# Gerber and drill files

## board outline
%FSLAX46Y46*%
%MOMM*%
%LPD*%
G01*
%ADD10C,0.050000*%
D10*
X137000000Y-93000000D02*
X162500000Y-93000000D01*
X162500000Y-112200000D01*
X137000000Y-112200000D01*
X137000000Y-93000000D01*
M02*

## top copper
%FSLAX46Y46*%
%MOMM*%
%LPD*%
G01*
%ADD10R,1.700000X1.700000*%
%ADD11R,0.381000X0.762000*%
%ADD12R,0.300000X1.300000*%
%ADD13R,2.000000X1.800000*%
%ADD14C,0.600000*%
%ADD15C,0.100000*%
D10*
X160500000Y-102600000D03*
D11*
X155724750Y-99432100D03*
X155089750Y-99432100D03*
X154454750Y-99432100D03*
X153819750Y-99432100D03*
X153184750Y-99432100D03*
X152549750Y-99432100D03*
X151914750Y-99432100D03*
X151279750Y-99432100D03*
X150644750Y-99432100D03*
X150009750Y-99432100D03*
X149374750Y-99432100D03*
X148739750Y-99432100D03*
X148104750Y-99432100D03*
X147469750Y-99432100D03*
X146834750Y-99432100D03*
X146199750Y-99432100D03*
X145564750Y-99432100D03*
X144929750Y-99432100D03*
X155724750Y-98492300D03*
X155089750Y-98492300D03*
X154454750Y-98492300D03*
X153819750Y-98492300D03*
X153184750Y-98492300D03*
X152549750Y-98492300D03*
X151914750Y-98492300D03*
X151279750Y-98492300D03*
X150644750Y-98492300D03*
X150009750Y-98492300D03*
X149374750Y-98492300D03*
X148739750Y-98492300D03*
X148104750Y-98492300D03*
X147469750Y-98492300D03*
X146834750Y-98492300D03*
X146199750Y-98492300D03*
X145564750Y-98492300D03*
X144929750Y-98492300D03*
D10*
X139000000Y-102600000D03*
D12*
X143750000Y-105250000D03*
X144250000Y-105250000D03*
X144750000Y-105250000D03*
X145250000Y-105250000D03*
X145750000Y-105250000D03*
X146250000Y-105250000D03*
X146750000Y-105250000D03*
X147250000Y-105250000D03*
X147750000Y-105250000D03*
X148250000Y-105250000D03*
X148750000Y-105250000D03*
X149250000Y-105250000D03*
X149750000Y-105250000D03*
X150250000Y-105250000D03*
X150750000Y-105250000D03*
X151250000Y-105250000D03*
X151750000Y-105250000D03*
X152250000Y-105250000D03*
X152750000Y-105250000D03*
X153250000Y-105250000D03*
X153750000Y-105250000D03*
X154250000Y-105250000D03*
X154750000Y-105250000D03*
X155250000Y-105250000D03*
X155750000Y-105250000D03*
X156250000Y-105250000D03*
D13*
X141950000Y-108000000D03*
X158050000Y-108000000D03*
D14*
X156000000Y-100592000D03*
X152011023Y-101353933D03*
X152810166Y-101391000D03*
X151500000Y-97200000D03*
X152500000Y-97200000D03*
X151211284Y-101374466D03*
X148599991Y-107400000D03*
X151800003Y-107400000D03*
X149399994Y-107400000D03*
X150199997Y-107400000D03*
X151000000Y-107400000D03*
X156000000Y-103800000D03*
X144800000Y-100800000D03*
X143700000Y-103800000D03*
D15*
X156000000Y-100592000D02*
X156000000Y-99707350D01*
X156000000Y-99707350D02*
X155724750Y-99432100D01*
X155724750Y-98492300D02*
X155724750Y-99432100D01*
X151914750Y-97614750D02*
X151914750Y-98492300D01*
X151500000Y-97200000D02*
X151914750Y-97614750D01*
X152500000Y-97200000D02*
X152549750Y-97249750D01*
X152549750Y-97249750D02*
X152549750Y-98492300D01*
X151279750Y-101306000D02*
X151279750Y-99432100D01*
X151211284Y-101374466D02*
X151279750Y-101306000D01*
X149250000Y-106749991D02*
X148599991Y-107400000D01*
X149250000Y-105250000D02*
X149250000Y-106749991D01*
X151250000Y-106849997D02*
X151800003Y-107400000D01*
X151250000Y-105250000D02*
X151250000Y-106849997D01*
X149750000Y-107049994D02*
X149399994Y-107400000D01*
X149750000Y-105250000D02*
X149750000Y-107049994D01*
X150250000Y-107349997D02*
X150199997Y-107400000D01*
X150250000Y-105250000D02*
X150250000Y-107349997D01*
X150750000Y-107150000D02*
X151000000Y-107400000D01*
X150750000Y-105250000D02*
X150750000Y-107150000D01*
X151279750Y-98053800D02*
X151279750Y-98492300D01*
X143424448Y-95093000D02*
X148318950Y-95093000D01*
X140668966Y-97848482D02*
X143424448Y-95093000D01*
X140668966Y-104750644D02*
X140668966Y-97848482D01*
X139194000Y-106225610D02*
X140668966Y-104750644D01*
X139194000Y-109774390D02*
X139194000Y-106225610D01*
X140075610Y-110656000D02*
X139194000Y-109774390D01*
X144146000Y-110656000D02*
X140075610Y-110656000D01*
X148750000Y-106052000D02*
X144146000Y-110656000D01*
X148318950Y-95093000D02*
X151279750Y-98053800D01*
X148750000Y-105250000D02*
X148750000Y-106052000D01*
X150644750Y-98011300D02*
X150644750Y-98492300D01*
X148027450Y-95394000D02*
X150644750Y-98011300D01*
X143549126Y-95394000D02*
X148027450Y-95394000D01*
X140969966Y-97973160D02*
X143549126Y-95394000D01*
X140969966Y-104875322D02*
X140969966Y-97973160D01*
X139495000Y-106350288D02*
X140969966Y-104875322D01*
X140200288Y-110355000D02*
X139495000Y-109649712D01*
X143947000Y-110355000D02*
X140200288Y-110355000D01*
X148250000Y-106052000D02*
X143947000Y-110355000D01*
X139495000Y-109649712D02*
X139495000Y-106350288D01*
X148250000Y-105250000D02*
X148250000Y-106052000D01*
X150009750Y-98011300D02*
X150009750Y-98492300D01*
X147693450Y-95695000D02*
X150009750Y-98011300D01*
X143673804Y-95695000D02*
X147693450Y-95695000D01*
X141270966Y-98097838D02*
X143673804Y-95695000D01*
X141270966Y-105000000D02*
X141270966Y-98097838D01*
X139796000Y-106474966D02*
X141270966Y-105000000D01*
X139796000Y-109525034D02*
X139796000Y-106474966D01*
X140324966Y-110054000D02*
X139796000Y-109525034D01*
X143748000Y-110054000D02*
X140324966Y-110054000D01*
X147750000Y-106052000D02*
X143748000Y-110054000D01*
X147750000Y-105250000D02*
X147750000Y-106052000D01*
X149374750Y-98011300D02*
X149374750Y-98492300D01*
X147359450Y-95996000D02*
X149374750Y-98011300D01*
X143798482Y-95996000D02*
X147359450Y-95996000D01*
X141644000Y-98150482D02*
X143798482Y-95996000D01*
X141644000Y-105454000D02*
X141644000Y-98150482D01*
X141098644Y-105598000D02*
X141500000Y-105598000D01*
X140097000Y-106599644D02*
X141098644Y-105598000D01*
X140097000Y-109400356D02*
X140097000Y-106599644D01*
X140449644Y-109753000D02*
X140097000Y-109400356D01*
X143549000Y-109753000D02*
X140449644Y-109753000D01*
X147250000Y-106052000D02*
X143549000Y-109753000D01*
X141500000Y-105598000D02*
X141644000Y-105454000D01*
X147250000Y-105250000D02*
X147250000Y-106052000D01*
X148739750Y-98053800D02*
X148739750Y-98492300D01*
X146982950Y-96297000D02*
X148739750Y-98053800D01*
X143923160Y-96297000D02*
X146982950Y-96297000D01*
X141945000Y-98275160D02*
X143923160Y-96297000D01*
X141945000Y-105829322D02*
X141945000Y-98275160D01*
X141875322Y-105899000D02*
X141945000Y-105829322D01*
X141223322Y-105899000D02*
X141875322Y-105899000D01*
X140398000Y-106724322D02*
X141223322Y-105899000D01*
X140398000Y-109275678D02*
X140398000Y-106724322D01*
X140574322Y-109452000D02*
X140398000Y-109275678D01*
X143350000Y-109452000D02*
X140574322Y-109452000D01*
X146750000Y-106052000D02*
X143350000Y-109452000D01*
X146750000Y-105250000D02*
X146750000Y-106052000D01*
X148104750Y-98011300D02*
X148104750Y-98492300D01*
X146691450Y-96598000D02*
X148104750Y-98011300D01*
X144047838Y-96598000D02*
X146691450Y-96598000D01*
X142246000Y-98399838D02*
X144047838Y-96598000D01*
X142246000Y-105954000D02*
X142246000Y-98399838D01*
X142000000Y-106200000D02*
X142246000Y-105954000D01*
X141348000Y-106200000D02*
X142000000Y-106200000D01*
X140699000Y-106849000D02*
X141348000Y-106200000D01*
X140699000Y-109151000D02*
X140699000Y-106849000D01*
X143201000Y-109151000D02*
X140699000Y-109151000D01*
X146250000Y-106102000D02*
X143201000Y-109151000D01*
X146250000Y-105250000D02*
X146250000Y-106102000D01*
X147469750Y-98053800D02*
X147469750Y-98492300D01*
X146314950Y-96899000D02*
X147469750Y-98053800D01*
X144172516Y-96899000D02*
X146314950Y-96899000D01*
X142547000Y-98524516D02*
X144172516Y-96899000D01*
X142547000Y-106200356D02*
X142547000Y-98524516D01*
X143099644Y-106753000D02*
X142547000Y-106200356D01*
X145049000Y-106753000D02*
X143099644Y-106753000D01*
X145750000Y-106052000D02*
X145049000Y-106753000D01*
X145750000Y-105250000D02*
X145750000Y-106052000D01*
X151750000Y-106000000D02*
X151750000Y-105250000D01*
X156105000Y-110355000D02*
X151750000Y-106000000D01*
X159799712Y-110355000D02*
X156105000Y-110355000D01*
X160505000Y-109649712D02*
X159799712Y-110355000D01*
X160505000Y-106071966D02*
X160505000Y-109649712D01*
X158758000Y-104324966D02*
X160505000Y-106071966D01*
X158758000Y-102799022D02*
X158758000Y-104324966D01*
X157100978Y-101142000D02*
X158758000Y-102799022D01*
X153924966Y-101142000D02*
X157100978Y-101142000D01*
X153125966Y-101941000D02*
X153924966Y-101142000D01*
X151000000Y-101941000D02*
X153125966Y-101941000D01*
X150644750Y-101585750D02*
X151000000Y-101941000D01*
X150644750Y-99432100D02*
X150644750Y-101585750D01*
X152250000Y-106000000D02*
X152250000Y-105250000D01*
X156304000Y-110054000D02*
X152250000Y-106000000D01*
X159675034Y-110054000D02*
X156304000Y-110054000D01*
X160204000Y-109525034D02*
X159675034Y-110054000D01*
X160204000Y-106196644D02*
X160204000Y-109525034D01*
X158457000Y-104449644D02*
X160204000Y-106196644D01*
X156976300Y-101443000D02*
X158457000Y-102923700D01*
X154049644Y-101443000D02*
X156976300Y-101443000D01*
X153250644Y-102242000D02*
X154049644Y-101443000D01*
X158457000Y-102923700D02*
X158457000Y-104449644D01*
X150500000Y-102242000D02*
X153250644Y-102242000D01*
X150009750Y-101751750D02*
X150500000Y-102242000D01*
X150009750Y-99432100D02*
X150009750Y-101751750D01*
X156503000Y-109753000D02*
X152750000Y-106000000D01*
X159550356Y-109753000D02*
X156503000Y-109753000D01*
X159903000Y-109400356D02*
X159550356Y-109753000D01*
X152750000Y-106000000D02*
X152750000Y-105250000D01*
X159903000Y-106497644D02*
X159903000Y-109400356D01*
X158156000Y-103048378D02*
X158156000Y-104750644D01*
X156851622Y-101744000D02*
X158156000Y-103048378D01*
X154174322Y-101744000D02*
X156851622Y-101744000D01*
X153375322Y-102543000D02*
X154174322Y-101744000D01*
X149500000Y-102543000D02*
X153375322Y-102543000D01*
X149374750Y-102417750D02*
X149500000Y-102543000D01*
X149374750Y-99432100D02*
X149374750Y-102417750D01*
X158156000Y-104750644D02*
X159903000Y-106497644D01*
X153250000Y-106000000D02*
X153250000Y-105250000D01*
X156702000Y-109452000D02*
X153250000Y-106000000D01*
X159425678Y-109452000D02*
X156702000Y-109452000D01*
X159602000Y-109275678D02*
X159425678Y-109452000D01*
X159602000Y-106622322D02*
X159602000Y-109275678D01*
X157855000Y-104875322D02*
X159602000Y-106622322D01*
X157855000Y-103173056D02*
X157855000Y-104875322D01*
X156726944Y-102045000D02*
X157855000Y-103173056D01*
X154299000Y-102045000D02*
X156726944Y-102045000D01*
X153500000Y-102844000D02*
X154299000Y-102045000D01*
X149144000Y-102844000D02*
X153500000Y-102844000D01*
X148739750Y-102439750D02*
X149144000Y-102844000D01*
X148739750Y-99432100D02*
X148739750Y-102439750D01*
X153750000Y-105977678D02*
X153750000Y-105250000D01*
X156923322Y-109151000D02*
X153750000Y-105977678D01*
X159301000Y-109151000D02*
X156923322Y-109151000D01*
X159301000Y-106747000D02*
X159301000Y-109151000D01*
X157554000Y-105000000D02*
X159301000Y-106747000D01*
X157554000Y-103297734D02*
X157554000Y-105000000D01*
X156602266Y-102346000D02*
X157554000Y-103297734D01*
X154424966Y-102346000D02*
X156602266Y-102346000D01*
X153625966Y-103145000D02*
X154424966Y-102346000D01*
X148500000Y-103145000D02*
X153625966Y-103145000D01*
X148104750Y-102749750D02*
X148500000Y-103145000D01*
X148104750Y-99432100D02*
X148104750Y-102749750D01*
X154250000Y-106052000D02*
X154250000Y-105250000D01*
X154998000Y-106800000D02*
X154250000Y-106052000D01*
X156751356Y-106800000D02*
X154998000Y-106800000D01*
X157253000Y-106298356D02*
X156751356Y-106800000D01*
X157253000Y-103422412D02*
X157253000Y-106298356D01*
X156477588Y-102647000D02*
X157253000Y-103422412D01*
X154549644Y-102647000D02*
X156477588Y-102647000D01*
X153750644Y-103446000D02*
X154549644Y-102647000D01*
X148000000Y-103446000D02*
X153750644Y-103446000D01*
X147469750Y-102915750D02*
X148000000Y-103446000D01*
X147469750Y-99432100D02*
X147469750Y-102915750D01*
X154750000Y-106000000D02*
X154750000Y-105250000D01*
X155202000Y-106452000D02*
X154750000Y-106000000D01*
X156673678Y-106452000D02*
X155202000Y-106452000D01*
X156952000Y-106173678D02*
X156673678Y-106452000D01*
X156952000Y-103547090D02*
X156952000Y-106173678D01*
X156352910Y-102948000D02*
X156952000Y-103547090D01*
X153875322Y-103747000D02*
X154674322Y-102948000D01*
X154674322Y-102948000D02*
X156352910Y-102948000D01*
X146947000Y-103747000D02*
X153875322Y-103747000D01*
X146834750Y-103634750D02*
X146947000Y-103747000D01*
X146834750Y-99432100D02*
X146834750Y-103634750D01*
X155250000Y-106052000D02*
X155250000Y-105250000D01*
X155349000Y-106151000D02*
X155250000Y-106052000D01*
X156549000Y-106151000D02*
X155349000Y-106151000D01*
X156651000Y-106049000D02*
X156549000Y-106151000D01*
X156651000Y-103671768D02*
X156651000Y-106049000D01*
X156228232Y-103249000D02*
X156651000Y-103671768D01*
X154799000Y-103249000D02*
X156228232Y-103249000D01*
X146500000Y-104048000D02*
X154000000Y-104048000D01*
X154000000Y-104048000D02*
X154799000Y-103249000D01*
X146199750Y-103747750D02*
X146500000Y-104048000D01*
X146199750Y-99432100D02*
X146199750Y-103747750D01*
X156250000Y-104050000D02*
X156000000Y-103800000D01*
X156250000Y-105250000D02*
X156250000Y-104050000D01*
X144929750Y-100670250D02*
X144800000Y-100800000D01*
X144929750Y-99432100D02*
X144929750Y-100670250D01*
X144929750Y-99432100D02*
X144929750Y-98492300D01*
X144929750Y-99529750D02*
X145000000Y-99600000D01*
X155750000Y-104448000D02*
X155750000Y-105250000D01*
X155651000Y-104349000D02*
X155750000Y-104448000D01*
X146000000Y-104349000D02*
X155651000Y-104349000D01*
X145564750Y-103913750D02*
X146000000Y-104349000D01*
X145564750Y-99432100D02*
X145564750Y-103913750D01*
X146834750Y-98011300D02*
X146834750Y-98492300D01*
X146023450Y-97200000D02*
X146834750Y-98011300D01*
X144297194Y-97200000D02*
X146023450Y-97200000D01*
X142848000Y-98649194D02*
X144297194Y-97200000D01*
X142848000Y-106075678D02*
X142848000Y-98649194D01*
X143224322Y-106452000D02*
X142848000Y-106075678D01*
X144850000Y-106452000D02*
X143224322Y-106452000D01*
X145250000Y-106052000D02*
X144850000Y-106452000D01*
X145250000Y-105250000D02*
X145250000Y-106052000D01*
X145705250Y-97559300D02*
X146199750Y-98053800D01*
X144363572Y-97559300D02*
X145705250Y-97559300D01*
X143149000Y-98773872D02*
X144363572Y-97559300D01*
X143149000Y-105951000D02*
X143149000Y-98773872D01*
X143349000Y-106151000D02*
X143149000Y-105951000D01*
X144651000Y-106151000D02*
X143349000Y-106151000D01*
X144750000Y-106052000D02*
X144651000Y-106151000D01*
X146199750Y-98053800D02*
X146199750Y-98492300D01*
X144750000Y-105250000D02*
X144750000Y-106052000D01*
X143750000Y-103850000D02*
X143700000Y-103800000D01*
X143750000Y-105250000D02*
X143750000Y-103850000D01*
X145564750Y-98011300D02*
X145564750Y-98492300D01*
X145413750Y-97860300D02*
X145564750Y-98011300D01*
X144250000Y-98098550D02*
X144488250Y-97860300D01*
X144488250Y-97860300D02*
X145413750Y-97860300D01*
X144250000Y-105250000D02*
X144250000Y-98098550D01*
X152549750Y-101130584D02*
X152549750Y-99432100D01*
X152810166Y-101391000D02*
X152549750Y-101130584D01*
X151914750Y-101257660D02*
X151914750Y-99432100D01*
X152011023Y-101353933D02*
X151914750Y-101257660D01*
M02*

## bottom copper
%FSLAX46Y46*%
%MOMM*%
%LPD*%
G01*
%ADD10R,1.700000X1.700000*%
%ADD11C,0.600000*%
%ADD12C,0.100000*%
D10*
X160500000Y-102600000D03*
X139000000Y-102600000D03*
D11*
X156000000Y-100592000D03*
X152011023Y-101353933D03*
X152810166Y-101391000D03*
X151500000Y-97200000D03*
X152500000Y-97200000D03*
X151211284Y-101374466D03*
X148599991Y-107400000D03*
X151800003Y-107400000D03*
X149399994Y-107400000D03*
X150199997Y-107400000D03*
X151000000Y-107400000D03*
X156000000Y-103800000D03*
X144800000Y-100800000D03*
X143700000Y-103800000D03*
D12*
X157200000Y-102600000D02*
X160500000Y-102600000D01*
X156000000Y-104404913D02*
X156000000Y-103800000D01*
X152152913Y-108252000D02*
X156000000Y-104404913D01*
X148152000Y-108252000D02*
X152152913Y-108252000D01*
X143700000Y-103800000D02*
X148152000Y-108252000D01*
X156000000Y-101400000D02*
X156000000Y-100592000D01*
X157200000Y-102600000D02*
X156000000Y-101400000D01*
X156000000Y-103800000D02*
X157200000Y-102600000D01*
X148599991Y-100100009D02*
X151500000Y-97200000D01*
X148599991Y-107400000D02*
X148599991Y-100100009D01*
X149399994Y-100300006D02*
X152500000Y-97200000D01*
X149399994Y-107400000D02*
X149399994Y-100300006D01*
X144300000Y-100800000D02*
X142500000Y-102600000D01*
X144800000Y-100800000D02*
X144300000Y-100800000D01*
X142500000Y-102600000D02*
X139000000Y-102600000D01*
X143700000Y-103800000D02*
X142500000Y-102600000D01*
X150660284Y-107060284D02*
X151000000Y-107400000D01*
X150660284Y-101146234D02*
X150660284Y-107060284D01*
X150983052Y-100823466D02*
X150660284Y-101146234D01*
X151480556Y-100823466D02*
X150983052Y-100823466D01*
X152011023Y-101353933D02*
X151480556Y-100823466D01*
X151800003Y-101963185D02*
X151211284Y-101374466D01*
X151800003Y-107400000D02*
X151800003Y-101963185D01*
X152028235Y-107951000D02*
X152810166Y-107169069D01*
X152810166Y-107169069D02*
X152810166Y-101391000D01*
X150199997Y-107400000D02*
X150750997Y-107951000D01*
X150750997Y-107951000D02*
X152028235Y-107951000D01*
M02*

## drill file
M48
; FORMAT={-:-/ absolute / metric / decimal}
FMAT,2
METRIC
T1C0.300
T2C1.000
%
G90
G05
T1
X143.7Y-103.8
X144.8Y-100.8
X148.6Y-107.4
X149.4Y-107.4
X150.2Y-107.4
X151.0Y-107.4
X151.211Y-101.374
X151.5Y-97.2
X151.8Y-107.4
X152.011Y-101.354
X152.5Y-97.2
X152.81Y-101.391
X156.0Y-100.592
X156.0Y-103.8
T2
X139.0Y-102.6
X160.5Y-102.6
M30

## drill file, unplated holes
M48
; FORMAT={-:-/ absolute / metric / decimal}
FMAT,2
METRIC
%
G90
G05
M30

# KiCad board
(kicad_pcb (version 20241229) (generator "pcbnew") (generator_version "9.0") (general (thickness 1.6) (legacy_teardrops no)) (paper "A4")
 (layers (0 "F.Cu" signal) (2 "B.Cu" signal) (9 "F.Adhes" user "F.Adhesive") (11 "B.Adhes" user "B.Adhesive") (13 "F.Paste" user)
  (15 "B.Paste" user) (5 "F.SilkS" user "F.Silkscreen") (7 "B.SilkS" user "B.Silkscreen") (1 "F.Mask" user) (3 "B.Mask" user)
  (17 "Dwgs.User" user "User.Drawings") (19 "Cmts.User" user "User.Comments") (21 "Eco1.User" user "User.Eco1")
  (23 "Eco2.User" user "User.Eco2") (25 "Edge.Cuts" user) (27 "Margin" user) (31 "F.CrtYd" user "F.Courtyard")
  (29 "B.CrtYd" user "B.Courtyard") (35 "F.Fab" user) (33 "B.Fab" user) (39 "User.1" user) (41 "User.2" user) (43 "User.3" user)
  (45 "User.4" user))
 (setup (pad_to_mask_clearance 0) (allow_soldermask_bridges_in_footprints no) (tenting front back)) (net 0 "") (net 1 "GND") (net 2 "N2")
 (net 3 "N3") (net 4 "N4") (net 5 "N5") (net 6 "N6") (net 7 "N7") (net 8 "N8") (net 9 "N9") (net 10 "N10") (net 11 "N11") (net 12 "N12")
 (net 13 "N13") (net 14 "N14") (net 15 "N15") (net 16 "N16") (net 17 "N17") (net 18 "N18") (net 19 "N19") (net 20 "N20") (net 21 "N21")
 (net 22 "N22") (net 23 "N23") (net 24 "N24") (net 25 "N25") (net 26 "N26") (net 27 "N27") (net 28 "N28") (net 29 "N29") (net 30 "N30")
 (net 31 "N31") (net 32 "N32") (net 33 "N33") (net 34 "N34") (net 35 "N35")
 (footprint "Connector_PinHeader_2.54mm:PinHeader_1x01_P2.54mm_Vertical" (layer "F.Cu") (at 139 102.6)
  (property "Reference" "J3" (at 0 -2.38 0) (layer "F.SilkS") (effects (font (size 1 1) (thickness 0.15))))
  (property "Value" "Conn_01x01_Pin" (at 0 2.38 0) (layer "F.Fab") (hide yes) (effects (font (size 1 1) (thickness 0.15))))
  (pad "1" thru_hole rect (at 0 0) (size 1.7 1.7) (drill 1) (layers "*.Cu" "*.Mask") (remove_unused_layers no) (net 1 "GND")))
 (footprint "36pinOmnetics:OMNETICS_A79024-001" (layer "F.Cu") (at 150.32725 98.9622 180)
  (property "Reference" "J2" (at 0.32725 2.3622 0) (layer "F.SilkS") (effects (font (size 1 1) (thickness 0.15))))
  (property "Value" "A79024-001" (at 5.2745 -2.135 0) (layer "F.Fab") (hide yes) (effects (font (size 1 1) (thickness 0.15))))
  (pad "1" smd rect (at 5.3975 0.4699 180) (size 0.381 0.762) (layers "F.Cu" "F.Mask" "F.Paste") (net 1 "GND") (solder_mask_margin 0.102))
  (pad "2" smd rect (at 4.7625 0.4699 180) (size 0.381 0.762) (layers "F.Cu" "F.Mask" "F.Paste") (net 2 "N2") (solder_mask_margin 0.102))
  (pad "3" smd rect (at 4.1275 0.4699 180) (size 0.381 0.762) (layers "F.Cu" "F.Mask" "F.Paste") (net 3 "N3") (solder_mask_margin 0.102))
  (pad "4" smd rect (at 3.4925 0.4699 180) (size 0.381 0.762) (layers "F.Cu" "F.Mask" "F.Paste") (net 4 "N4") (solder_mask_margin 0.102))
  (pad "5" smd rect (at 2.8575 0.4699 180) (size 0.381 0.762) (layers "F.Cu" "F.Mask" "F.Paste") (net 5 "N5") (solder_mask_margin 0.102))
  (pad "6" smd rect (at 2.2225 0.4699 180) (size 0.381 0.762) (layers "F.Cu" "F.Mask" "F.Paste") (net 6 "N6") (solder_mask_margin 0.102))
  (pad "7" smd rect (at 1.5875 0.4699 180) (size 0.381 0.762) (layers "F.Cu" "F.Mask" "F.Paste") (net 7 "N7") (solder_mask_margin 0.102))
  (pad "8" smd rect (at 0.9525 0.4699 180) (size 0.381 0.762) (layers "F.Cu" "F.Mask" "F.Paste") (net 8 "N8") (solder_mask_margin 0.102))
  (pad "9" smd rect (at 0.3175 0.4699 180) (size 0.381 0.762) (layers "F.Cu" "F.Mask" "F.Paste") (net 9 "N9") (solder_mask_margin 0.102))
  (pad "10" smd rect (at -0.3175 0.4699 180) (size 0.381 0.762) (layers "F.Cu" "F.Mask" "F.Paste") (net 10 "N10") (solder_mask_margin 0.102))
  (pad "11" smd rect (at -0.9525 0.4699 180) (size 0.381 0.762) (layers "F.Cu" "F.Mask" "F.Paste") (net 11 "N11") (solder_mask_margin 0.102))
  (pad "12" smd rect (at -1.5875 0.4699 180) (size 0.381 0.762) (layers "F.Cu" "F.Mask" "F.Paste") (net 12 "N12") (solder_mask_margin 0.102))
  (pad "13" smd rect (at -2.2225 0.4699 180) (size 0.381 0.762) (layers "F.Cu" "F.Mask" "F.Paste") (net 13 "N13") (solder_mask_margin 0.102))
  (pad "14" smd rect (at -2.8575 0.4699 180) (size 0.381 0.762) (layers "F.Cu" "F.Mask" "F.Paste") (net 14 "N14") (solder_mask_margin 0.102))
  (pad "15" smd rect (at -3.4925 0.4699 180) (size 0.381 0.762) (layers "F.Cu" "F.Mask" "F.Paste") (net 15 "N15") (solder_mask_margin 0.102))
  (pad "16" smd rect (at -4.1275 0.4699 180) (size 0.381 0.762) (layers "F.Cu" "F.Mask" "F.Paste") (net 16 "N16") (solder_mask_margin 0.102))
  (pad "17" smd rect (at -4.7625 0.4699 180) (size 0.381 0.762) (layers "F.Cu" "F.Mask" "F.Paste") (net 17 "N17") (solder_mask_margin 0.102))
  (pad "18" smd rect (at -5.3975 0.4699 180) (size 0.381 0.762) (layers "F.Cu" "F.Mask" "F.Paste") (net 1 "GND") (solder_mask_margin 0.102))
  (pad "19" smd rect (at 5.3975 -0.4699 180) (size 0.381 0.762) (layers "F.Cu" "F.Mask" "F.Paste") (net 1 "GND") (solder_mask_margin 0.102))
  (pad "20" smd rect (at 4.7625 -0.4699 180) (size 0.381 0.762) (layers "F.Cu" "F.Mask" "F.Paste") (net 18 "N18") (solder_mask_margin 0.102))
  (pad "21" smd rect (at 4.1275 -0.4699 180) (size 0.381 0.762) (layers "F.Cu" "F.Mask" "F.Paste") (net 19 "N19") (solder_mask_margin 0.102))
  (pad "22" smd rect (at 3.4925 -0.4699 180) (size 0.381 0.762) (layers "F.Cu" "F.Mask" "F.Paste") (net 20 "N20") (solder_mask_margin 0.102))
  (pad "23" smd rect (at 2.8575 -0.4699 180) (size 0.381 0.762) (layers "F.Cu" "F.Mask" "F.Paste") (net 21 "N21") (solder_mask_margin 0.102))
  (pad "24" smd rect (at 2.2225 -0.4699 180) (size 0.381 0.762) (layers "F.Cu" "F.Mask" "F.Paste") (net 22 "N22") (solder_mask_margin 0.102))
  (pad "25" smd rect (at 1.5875 -0.4699 180) (size 0.381 0.762) (layers "F.Cu" "F.Mask" "F.Paste") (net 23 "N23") (solder_mask_margin 0.102))
  (pad "26" smd rect (at 0.9525 -0.4699 180) (size 0.381 0.762) (layers "F.Cu" "F.Mask" "F.Paste") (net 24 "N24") (solder_mask_margin 0.102))
  (pad "27" smd rect (at 0.3175 -0.4699 180) (size 0.381 0.762) (layers "F.Cu" "F.Mask" "F.Paste") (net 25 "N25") (solder_mask_margin 0.102))
  (pad "28" smd rect (at -0.3175 -0.4699 180) (size 0.381 0.762) (layers "F.Cu" "F.Mask" "F.Paste") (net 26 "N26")
   (solder_mask_margin 0.102))
  (pad "29" smd rect (at -0.9525 -0.4699 180) (size 0.381 0.762) (layers "F.Cu" "F.Mask" "F.Paste") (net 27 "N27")
   (solder_mask_margin 0.102))
  (pad "30" smd rect (at -1.5875 -0.4699 180) (size 0.381 0.762) (layers "F.Cu" "F.Mask" "F.Paste") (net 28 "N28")
   (solder_mask_margin 0.102))
  (pad "31" smd rect (at -2.2225 -0.4699 180) (size 0.381 0.762) (layers "F.Cu" "F.Mask" "F.Paste") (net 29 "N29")
   (solder_mask_margin 0.102))
  (pad "32" smd rect (at -2.8575 -0.4699 180) (size 0.381 0.762) (layers "F.Cu" "F.Mask" "F.Paste") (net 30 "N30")
   (solder_mask_margin 0.102))
  (pad "33" smd rect (at -3.4925 -0.4699 180) (size 0.381 0.762) (layers "F.Cu" "F.Mask" "F.Paste") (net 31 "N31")
   (solder_mask_margin 0.102))
  (pad "34" smd rect (at -4.1275 -0.4699 180) (size 0.381 0.762) (layers "F.Cu" "F.Mask" "F.Paste") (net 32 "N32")
   (solder_mask_margin 0.102))
  (pad "35" smd rect (at -4.7625 -0.4699 180) (size 0.381 0.762) (layers "F.Cu" "F.Mask" "F.Paste") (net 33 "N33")
   (solder_mask_margin 0.102))
  (pad "36" smd rect (at -5.3975 -0.4699 180) (size 0.381 0.762) (layers "F.Cu" "F.Mask" "F.Paste") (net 1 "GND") (solder_mask_margin 0.102)))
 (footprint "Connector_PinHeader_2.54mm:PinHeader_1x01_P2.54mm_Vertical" (layer "F.Cu") (at 160.5 102.6)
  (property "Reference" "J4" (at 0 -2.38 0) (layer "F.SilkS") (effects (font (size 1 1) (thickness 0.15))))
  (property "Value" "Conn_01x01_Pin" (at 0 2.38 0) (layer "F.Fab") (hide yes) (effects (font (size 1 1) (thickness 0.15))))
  (pad "1" thru_hole rect (at 0 0) (size 1.7 1.7) (drill 1) (layers "*.Cu" "*.Mask") (remove_unused_layers no) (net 1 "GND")))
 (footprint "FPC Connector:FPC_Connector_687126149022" (layer "F.Cu") (at 150 108.6)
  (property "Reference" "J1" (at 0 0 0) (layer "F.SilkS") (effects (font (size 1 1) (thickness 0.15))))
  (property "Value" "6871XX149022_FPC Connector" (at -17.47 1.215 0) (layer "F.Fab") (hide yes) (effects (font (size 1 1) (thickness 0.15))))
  (pad "1" smd rect (at -6.25 -3.35) (size 0.3 1.3) (layers "F.Cu" "F.Mask" "F.Paste") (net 1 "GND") (solder_mask_margin 0.102))
  (pad "2" smd rect (at -5.75 -3.35) (size 0.3 1.3) (layers "F.Cu" "F.Mask" "F.Paste") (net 2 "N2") (solder_mask_margin 0.102))
  (pad "3" smd rect (at -5.25 -3.35) (size 0.3 1.3) (layers "F.Cu" "F.Mask" "F.Paste") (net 3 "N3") (solder_mask_margin 0.102))
  (pad "4" smd rect (at -4.75 -3.35) (size 0.3 1.3) (layers "F.Cu" "F.Mask" "F.Paste") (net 4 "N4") (solder_mask_margin 0.102))
  (pad "5" smd rect (at -4.25 -3.35) (size 0.3 1.3) (layers "F.Cu" "F.Mask" "F.Paste") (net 5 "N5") (solder_mask_margin 0.102))
  (pad "6" smd rect (at -3.75 -3.35) (size 0.3 1.3) (layers "F.Cu" "F.Mask" "F.Paste") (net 6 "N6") (solder_mask_margin 0.102))
  (pad "7" smd rect (at -3.25 -3.35) (size 0.3 1.3) (layers "F.Cu" "F.Mask" "F.Paste") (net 7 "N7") (solder_mask_margin 0.102))
  (pad "8" smd rect (at -2.75 -3.35) (size 0.3 1.3) (layers "F.Cu" "F.Mask" "F.Paste") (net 8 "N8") (solder_mask_margin 0.102))
  (pad "9" smd rect (at -2.25 -3.35) (size 0.3 1.3) (layers "F.Cu" "F.Mask" "F.Paste") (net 9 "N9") (solder_mask_margin 0.102))
  (pad "10" smd rect (at -1.75 -3.35) (size 0.3 1.3) (layers "F.Cu" "F.Mask" "F.Paste") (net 10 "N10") (solder_mask_margin 0.102))
  (pad "11" smd rect (at -1.25 -3.35) (size 0.3 1.3) (layers "F.Cu" "F.Mask" "F.Paste") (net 11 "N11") (solder_mask_margin 0.102))
  (pad "12" smd rect (at -0.75 -3.35) (size 0.3 1.3) (layers "F.Cu" "F.Mask" "F.Paste") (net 12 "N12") (solder_mask_margin 0.102))
  (pad "13" smd rect (at -0.25 -3.35) (size 0.3 1.3) (layers "F.Cu" "F.Mask" "F.Paste") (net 13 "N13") (solder_mask_margin 0.102))
  (pad "14" smd rect (at 0.25 -3.35) (size 0.3 1.3) (layers "F.Cu" "F.Mask" "F.Paste") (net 29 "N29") (solder_mask_margin 0.102))
  (pad "15" smd rect (at 0.75 -3.35) (size 0.3 1.3) (layers "F.Cu" "F.Mask" "F.Paste") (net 28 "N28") (solder_mask_margin 0.102))
  (pad "16" smd rect (at 1.25 -3.35) (size 0.3 1.3) (layers "F.Cu" "F.Mask" "F.Paste") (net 27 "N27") (solder_mask_margin 0.102))
  (pad "17" smd rect (at 1.75 -3.35) (size 0.3 1.3) (layers "F.Cu" "F.Mask" "F.Paste") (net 26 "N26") (solder_mask_margin 0.102))
  (pad "18" smd rect (at 2.25 -3.35) (size 0.3 1.3) (layers "F.Cu" "F.Mask" "F.Paste") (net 25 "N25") (solder_mask_margin 0.102))
  (pad "19" smd rect (at 2.75 -3.35) (size 0.3 1.3) (layers "F.Cu" "F.Mask" "F.Paste") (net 24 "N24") (solder_mask_margin 0.102))
  (pad "20" smd rect (at 3.25 -3.35) (size 0.3 1.3) (layers "F.Cu" "F.Mask" "F.Paste") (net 23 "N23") (solder_mask_margin 0.102))
  (pad "21" smd rect (at 3.75 -3.35) (size 0.3 1.3) (layers "F.Cu" "F.Mask" "F.Paste") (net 22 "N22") (solder_mask_margin 0.102))
  (pad "22" smd rect (at 4.25 -3.35) (size 0.3 1.3) (layers "F.Cu" "F.Mask" "F.Paste") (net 21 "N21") (solder_mask_margin 0.102))
  (pad "23" smd rect (at 4.75 -3.35) (size 0.3 1.3) (layers "F.Cu" "F.Mask" "F.Paste") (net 20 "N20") (solder_mask_margin 0.102))
  (pad "24" smd rect (at 5.25 -3.35) (size 0.3 1.3) (layers "F.Cu" "F.Mask" "F.Paste") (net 19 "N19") (solder_mask_margin 0.102))
  (pad "25" smd rect (at 5.75 -3.35) (size 0.3 1.3) (layers "F.Cu" "F.Mask" "F.Paste") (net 18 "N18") (solder_mask_margin 0.102))
  (pad "26" smd rect (at 6.25 -3.35) (size 0.3 1.3) (layers "F.Cu" "F.Mask" "F.Paste") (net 1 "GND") (solder_mask_margin 0.102))
  (pad "Z1" smd rect (at -8.05 -0.6) (size 2 1.8) (layers "F.Cu" "F.Mask" "F.Paste") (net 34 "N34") (solder_mask_margin 0.102))
  (pad "Z2" smd rect (at 8.05 -0.6) (size 2 1.8) (layers "F.Cu" "F.Mask" "F.Paste") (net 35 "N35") (solder_mask_margin 0.102)))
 (gr_rect (start 137 93) (end 162.5 112.2) (stroke (width 0.05) (type default)) (fill no) (layer "Edge.Cuts"))
 (segment (start 140.969966 97.97316) (end 143.549126 95.394) (width 0.1) (layer "F.Cu") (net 10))
 (segment (start 140.969966 104.875322) (end 140.969966 97.97316) (width 0.1) (layer "F.Cu") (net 10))
 (segment (start 140.200288 110.355) (end 139.495 109.649712) (width 0.1) (layer "F.Cu") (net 10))
 (segment (start 143.947 110.355) (end 140.200288 110.355) (width 0.1) (layer "F.Cu") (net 10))
 (segment (start 139.495 109.649712) (end 139.495 106.350288) (width 0.1) (layer "F.Cu") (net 10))
 (segment (start 148.25 106.052) (end 143.947 110.355) (width 0.1) (layer "F.Cu") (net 10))
 (segment (start 143.549126 95.394) (end 148.02745 95.394) (width 0.1) (layer "F.Cu") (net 10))
 (segment (start 148.02745 95.394) (end 150.64475 98.0113) (width 0.1) (layer "F.Cu") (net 10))
 (segment (start 139.495 106.350288) (end 140.969966 104.875322) (width 0.1) (layer "F.Cu") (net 10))
 (segment (start 148.25 105.25) (end 148.25 106.052) (width 0.1) (layer "F.Cu") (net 10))
 (segment (start 150.64475 98.0113) (end 150.64475 98.4923) (width 0.1) (layer "F.Cu") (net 10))
 (segment (start 150.00975 98.0113) (end 150.00975 98.4923) (width 0.1) (layer "F.Cu") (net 9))
 (segment (start 141.270966 105) (end 141.270966 98.097838) (width 0.1) (layer "F.Cu") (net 9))
 (segment (start 147.75 106.052) (end 143.748 110.054) (width 0.1) (layer "F.Cu") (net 9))
 (segment (start 140.324966 110.054) (end 139.796 109.525034) (width 0.1) (layer "F.Cu") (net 9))
 (segment (start 143.748 110.054) (end 140.324966 110.054) (width 0.1) (layer "F.Cu") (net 9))
 (segment (start 147.75 105.25) (end 147.75 106.052) (width 0.1) (layer "F.Cu") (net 9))
 (segment (start 143.673804 95.695) (end 147.69345 95.695) (width 0.1) (layer "F.Cu") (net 9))
 (segment (start 147.69345 95.695) (end 150.00975 98.0113) (width 0.1) (layer "F.Cu") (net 9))
 (segment (start 141.270966 98.097838) (end 143.673804 95.695) (width 0.1) (layer "F.Cu") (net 9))
 (segment (start 139.796 106.474966) (end 141.270966 105) (width 0.1) (layer "F.Cu") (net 9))
 (segment (start 139.796 109.525034) (end 139.796 106.474966) (width 0.1) (layer "F.Cu") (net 9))
 (segment (start 151.27975 101.306) (end 151.27975 99.4321) (width 0.1) (layer "F.Cu") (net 27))
 (segment (start 151.211284 101.374466) (end 151.27975 101.306) (width 0.1) (layer "F.Cu") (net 27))
 (segment (start 151.25 106.849997) (end 151.800003 107.4) (width 0.1) (layer "F.Cu") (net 27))
 (segment (start 151.25 105.25) (end 151.25 106.849997) (width 0.1) (layer "F.Cu") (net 27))
 (via (at 151.800003 107.4) (size 0.6) (drill 0.3) (layers "F.Cu" "B.Cu") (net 27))
 (via (at 151.211284 101.374466) (size 0.6) (drill 0.3) (layers "F.Cu" "B.Cu") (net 27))
 (segment (start 151.800003 107.4) (end 151.800003 101.963185) (width 0.1) (layer "B.Cu") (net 27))
 (segment (start 151.800003 101.963185) (end 151.211284 101.374466) (width 0.1) (layer "B.Cu") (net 27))
 (segment (start 140.398 106.724322) (end 141.223322 105.899) (width 0.1) (layer "F.Cu") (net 7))
 (segment (start 146.75 105.25) (end 146.75 106.052) (width 0.1) (layer "F.Cu") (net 7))
 (segment (start 146.98295 96.297) (end 148.73975 98.0538) (width 0.1) (layer "F.Cu") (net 7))
 (segment (start 146.75 106.052) (end 143.35 109.452) (width 0.1) (layer "F.Cu") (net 7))
 (segment (start 143.92316 96.297) (end 146.98295 96.297) (width 0.1) (layer "F.Cu") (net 7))
 (segment (start 141.945 98.27516) (end 143.92316 96.297) (width 0.1) (layer "F.Cu") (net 7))
 (segment (start 141.875322 105.899) (end 141.945 105.829322) (width 0.1) (layer "F.Cu") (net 7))
 (segment (start 141.223322 105.899) (end 141.875322 105.899) (width 0.1) (layer "F.Cu") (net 7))
 (segment (start 140.398 109.275678) (end 140.398 106.724322) (width 0.1) (layer "F.Cu") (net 7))
 (segment (start 143.35 109.452) (end 140.574322 109.452) (width 0.1) (layer "F.Cu") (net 7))
 (segment (start 141.945 105.829322) (end 141.945 98.27516) (width 0.1) (layer "F.Cu") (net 7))
 (segment (start 148.73975 98.0538) (end 148.73975 98.4923) (width 0.1) (layer "F.Cu") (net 7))
 (segment (start 140.574322 109.452) (end 140.398 109.275678) (width 0.1) (layer "F.Cu") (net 7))
 (segment (start 152.810166 101.391) (end 152.54975 101.130584) (width 0.1) (layer "F.Cu") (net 29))
 (segment (start 152.54975 101.130584) (end 152.54975 99.4321) (width 0.1) (layer "F.Cu") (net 29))
 (segment (start 150.25 107.349997) (end 150.199997 107.4) (width 0.1) (layer "F.Cu") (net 29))
 (segment (start 150.25 105.25) (end 150.25 107.349997) (width 0.1) (layer "F.Cu") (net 29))
 (via (at 152.810166 101.391) (size 0.6) (drill 0.3) (layers "F.Cu" "B.Cu") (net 29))
 (via (at 150.199997 107.4) (size 0.6) (drill 0.3) (layers "F.Cu" "B.Cu") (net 29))
 (segment (start 152.028235 107.951) (end 152.810166 107.169069) (width 0.1) (layer "B.Cu") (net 29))
 (segment (start 150.199997 107.4) (end 150.750997 107.951) (width 0.1) (layer "B.Cu") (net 29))
 (segment (start 150.750997 107.951) (end 152.028235 107.951) (width 0.1) (layer "B.Cu") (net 29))
 (segment (start 152.810166 107.169069) (end 152.810166 101.391) (width 0.1) (layer "B.Cu") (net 29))
 (segment (start 144.25 105.25) (end 144.25 98.09855) (width 0.1) (layer "F.Cu") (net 2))
 (segment (start 144.48825 97.8603) (end 145.41375 97.8603) (width 0.1) (layer "F.Cu") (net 2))
 (segment (start 144.25 98.09855) (end 144.48825 97.8603) (width 0.1) (layer "F.Cu") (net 2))
 (segment (start 145.56475 98.0113) (end 145.56475 98.4923) (width 0.1) (layer "F.Cu") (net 2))
 (segment (start 145.41375 97.8603) (end 145.56475 98.0113) (width 0.1) (layer "F.Cu") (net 2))
 (segment (start 146.31495 96.899) (end 147.46975 98.0538) (width 0.1) (layer "F.Cu") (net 5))
 (segment (start 142.547 98.524516) (end 144.172516 96.899) (width 0.1) (layer "F.Cu") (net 5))
 (segment (start 144.172516 96.899) (end 146.31495 96.899) (width 0.1) (layer "F.Cu") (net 5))
 (segment (start 145.049 106.753) (end 143.099644 106.753) (width 0.1) (layer "F.Cu") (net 5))
 (segment (start 143.099644 106.753) (end 142.547 106.200356) (width 0.1) (layer "F.Cu") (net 5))
 (segment (start 145.75 106.052) (end 145.049 106.753) (width 0.1) (layer "F.Cu") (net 5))
 (segment (start 147.46975 98.0538) (end 147.46975 98.4923) (width 0.1) (layer "F.Cu") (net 5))
 (segment (start 145.75 105.25) (end 145.75 106.052) (width 0.1) (layer "F.Cu") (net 5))
 (segment (start 142.547 106.200356) (end 142.547 98.524516) (width 0.1) (layer "F.Cu") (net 5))
 (segment (start 142.246 105.954) (end 142.246 98.399838) (width 0.1) (layer "F.Cu") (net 6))
 (segment (start 146.25 105.25) (end 146.25 106.102) (width 0.1) (layer "F.Cu") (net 6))
 (segment (start 143.201 109.151) (end 140.699 109.151) (width 0.1) (layer "F.Cu") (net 6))
 (segment (start 146.25 106.102) (end 143.201 109.151) (width 0.1) (layer "F.Cu") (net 6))
 (segment (start 142.246 98.399838) (end 144.047838 96.598) (width 0.1) (layer "F.Cu") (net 6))
 (segment (start 140.699 106.849) (end 141.348 106.2) (width 0.1) (layer "F.Cu") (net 6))
 (segment (start 146.69145 96.598) (end 148.10475 98.0113) (width 0.1) (layer "F.Cu") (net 6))
 (segment (start 144.047838 96.598) (end 146.69145 96.598) (width 0.1) (layer "F.Cu") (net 6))
 (segment (start 142 106.2) (end 142.246 105.954) (width 0.1) (layer "F.Cu") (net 6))
 (segment (start 141.348 106.2) (end 142 106.2) (width 0.1) (layer "F.Cu") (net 6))
 (segment (start 148.10475 98.0113) (end 148.10475 98.4923) (width 0.1) (layer "F.Cu") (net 6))
 (segment (start 140.699 109.151) (end 140.699 106.849) (width 0.1) (layer "F.Cu") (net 6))
 (segment (start 146.947 103.747) (end 153.875322 103.747) (width 0.1) (layer "F.Cu") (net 20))
 (segment (start 146.83475 99.4321) (end 146.83475 103.63475) (width 0.1) (layer "F.Cu") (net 20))
 (segment (start 156.952 103.54709) (end 156.952 106.173678) (width 0.1) (layer "F.Cu") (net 20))
 (segment (start 156.952 106.173678) (end 156.673678 106.452) (width 0.1) (layer "F.Cu") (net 20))
 (segment (start 155.202 106.452) (end 154.75 106) (width 0.1) (layer "F.Cu") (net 20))
 (segment (start 154.75 106) (end 154.75 105.25) (width 0.1) (layer "F.Cu") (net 20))
 (segment (start 146.83475 103.63475) (end 146.947 103.747) (width 0.1) (layer "F.Cu") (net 20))
 (segment (start 156.35291 102.948) (end 156.952 103.54709) (width 0.1) (layer "F.Cu") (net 20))
 (segment (start 153.875322 103.747) (end 154.674322 102.948) (width 0.1) (layer "F.Cu") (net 20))
 (segment (start 154.674322 102.948) (end 156.35291 102.948) (width 0.1) (layer "F.Cu") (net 20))
 (segment (start 156.673678 106.452) (end 155.202 106.452) (width 0.1) (layer "F.Cu") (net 20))
 (segment (start 153.375322 102.543) (end 154.174322 101.744) (width 0.1) (layer "F.Cu") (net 24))
 (segment (start 149.37475 102.41775) (end 149.5 102.543) (width 0.1) (layer "F.Cu") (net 24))
 (segment (start 156.503 109.753) (end 152.75 106) (width 0.1) (layer "F.Cu") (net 24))
 (segment (start 156.851622 101.744) (end 158.156 103.048378) (width 0.1) (layer "F.Cu") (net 24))
 (segment (start 154.174322 101.744) (end 156.851622 101.744) (width 0.1) (layer "F.Cu") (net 24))
 (segment (start 159.903 106.497644) (end 159.903 109.400356) (width 0.1) (layer "F.Cu") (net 24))
 (segment (start 149.37475 99.4321) (end 149.37475 102.41775) (width 0.1) (layer "F.Cu") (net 24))
 (segment (start 158.156 104.750644) (end 159.903 106.497644) (width 0.1) (layer "F.Cu") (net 24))
 (segment (start 152.75 106) (end 152.75 105.25) (width 0.1) (layer "F.Cu") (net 24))
 (segment (start 159.903 109.400356) (end 159.550356 109.753) (width 0.1) (layer "F.Cu") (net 24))
 (segment (start 149.5 102.543) (end 153.375322 102.543) (width 0.1) (layer "F.Cu") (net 24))
 (segment (start 159.550356 109.753) (end 156.503 109.753) (width 0.1) (layer "F.Cu") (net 24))
 (segment (start 158.156 103.048378) (end 158.156 104.750644) (width 0.1) (layer "F.Cu") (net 24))
 (segment (start 143.75 103.85) (end 143.7 103.8) (width 0.1) (layer "F.Cu") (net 1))
 (segment (start 143.75 105.25) (end 143.75 103.85) (width 0.1) (layer "F.Cu") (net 1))
 (segment (start 156.25 104.05) (end 156 103.8) (width 0.1) (layer "F.Cu") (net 1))
 (segment (start 144.92975 99.52975) (end 145 99.6) (width 0.1) (layer "F.Cu") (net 1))
 (segment (start 156 99.70735) (end 155.72475 99.4321) (width 0.1) (layer "F.Cu") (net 1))
 (segment (start 144.92975 99.4321) (end 144.92975 98.4923) (width 0.1) (layer "F.Cu") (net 1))
 (segment (start 155.72475 98.4923) (end 155.72475 99.4321) (width 0.1) (layer "F.Cu") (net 1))
 (segment (start 144.92975 100.67025) (end 144.8 100.8) (width 0.1) (layer "F.Cu") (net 1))
 (segment (start 156 100.592) (end 156 99.70735) (width 0.1) (layer "F.Cu") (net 1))
 (segment (start 156.25 105.25) (end 156.25 104.05) (width 0.1) (layer "F.Cu") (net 1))
 (segment (start 144.92975 99.4321) (end 144.92975 100.67025) (width 0.1) (layer "F.Cu") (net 1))
 (via (at 143.7 103.8) (size 0.6) (drill 0.3) (layers "F.Cu" "B.Cu") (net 1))
 (via (at 144.8 100.8) (size 0.6) (drill 0.3) (layers "F.Cu" "B.Cu") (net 1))
 (via (at 156 103.8) (size 0.6) (drill 0.3) (layers "F.Cu" "B.Cu") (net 1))
 (via (at 156 100.592) (size 0.6) (drill 0.3) (layers "F.Cu" "B.Cu") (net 1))
 (segment (start 144.3 100.8) (end 142.5 102.6) (width 0.1) (layer "B.Cu") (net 1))
 (segment (start 156 101.4) (end 156 100.592) (width 0.1) (layer "B.Cu") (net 1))
 (segment (start 144.8 100.8) (end 144.3 100.8) (width 0.1) (layer "B.Cu") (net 1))
 (segment (start 143.7 103.8) (end 142.5 102.6) (width 0.1) (layer "B.Cu") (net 1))
 (segment (start 156 103.8) (end 157.2 102.6) (width 0.1) (layer "B.Cu") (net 1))
 (segment (start 157.2 102.6) (end 160.5 102.6) (width 0.1) (layer "B.Cu") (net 1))
 (segment (start 143.7 103.8) (end 148.152 108.252) (width 0.1) (layer "B.Cu") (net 1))
 (segment (start 152.152913 108.252) (end 156 104.404913) (width 0.1) (layer "B.Cu") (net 1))
 (segment (start 156 104.404913) (end 156 103.8) (width 0.1) (layer "B.Cu") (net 1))
 (segment (start 157.2 102.6) (end 156 101.4) (width 0.1) (layer "B.Cu") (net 1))
 (segment (start 142.5 102.6) (end 139 102.6) (width 0.1) (layer "B.Cu") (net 1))
 (segment (start 148.152 108.252) (end 152.152913 108.252) (width 0.1) (layer "B.Cu") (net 1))
 (segment (start 146.83475 98.0113) (end 146.83475 98.4923) (width 0.1) (layer "F.Cu") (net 4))
 (segment (start 142.848 106.075678) (end 142.848 98.649194) (width 0.1) (layer "F.Cu") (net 4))
 (segment (start 145.25 106.052) (end 144.85 106.452) (width 0.1) (layer "F.Cu") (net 4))
 (segment (start 146.02345 97.2) (end 146.83475 98.0113) (width 0.1) (layer "F.Cu") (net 4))
 (segment (start 145.25 105.25) (end 145.25 106.052) (width 0.1) (layer "F.Cu") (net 4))
 (segment (start 144.297194 97.2) (end 146.02345 97.2) (width 0.1) (layer "F.Cu") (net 4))
 (segment (start 142.848 98.649194) (end 144.297194 97.2) (width 0.1) (layer "F.Cu") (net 4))
 (segment (start 144.85 106.452) (end 143.224322 106.452) (width 0.1) (layer "F.Cu") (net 4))
 (segment (start 143.224322 106.452) (end 142.848 106.075678) (width 0.1) (layer "F.Cu") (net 4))
 (segment (start 152.011023 101.353933) (end 151.91475 101.25766) (width 0.1) (layer "F.Cu") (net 28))
 (segment (start 150.75 107.15) (end 151 107.4) (width 0.1) (layer "F.Cu") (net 28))
 (segment (start 150.75 105.25) (end 150.75 107.15) (width 0.1) (layer "F.Cu") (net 28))
 (segment (start 151.91475 101.25766) (end 151.91475 99.4321) (width 0.1) (layer "F.Cu") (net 28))
 (via (at 151 107.4) (size 0.6) (drill 0.3) (layers "F.Cu" "B.Cu") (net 28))
 (via (at 152.011023 101.353933) (size 0.6) (drill 0.3) (layers "F.Cu" "B.Cu") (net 28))
 (segment (start 150.660284 107.060284) (end 151 107.4) (width 0.1) (layer "B.Cu") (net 28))
 (segment (start 151.480556 100.823466) (end 150.983052 100.823466) (width 0.1) (layer "B.Cu") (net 28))
 (segment (start 152.011023 101.353933) (end 151.480556 100.823466) (width 0.1) (layer "B.Cu") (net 28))
 (segment (start 150.983052 100.823466) (end 150.660284 101.146234) (width 0.1) (layer "B.Cu") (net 28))
 (segment (start 150.660284 101.146234) (end 150.660284 107.060284) (width 0.1) (layer "B.Cu") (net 28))
 (segment (start 151.5 97.2) (end 151.91475 97.61475) (width 0.1) (layer "F.Cu") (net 12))
 (segment (start 149.25 105.25) (end 149.25 106.749991) (width 0.1) (layer "F.Cu") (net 12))
 (segment (start 149.25 106.749991) (end 148.599991 107.4) (width 0.1) (layer "F.Cu") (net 12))
 (segment (start 151.91475 97.61475) (end 151.91475 98.4923) (width 0.1) (layer "F.Cu") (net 12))
 (via (at 148.599991 107.4) (size 0.6) (drill 0.3) (layers "F.Cu" "B.Cu") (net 12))
 (via (at 151.5 97.2) (size 0.6) (drill 0.3) (layers "F.Cu" "B.Cu") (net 12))
 (segment (start 148.599991 107.4) (end 148.599991 100.100009) (width 0.1) (layer "B.Cu") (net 12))
 (segment (start 148.599991 100.100009) (end 151.5 97.2) (width 0.1) (layer "B.Cu") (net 12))
 (segment (start 159.675034 110.054) (end 156.304 110.054) (width 0.1) (layer "F.Cu") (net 25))
 (segment (start 150.00975 99.4321) (end 150.00975 101.75175) (width 0.1) (layer "F.Cu") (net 25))
 (segment (start 150.00975 101.75175) (end 150.5 102.242) (width 0.1) (layer "F.Cu") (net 25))
 (segment (start 160.204 109.525034) (end 159.675034 110.054) (width 0.1) (layer "F.Cu") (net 25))
 (segment (start 154.049644 101.443) (end 156.9763 101.443) (width 0.1) (layer "F.Cu") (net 25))
 (segment (start 160.204 106.196644) (end 160.204 109.525034) (width 0.1) (layer "F.Cu") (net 25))
 (segment (start 153.250644 102.242) (end 154.049644 101.443) (width 0.1) (layer "F.Cu") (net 25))
 (segment (start 156.304 110.054) (end 152.25 106) (width 0.1) (layer "F.Cu") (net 25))
 (segment (start 150.5 102.242) (end 153.250644 102.242) (width 0.1) (layer "F.Cu") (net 25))
 (segment (start 158.457 104.449644) (end 160.204 106.196644) (width 0.1) (layer "F.Cu") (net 25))
 (segment (start 156.9763 101.443) (end 158.457 102.9237) (width 0.1) (layer "F.Cu") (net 25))
 (segment (start 152.25 106) (end 152.25 105.25) (width 0.1) (layer "F.Cu") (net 25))
 (segment (start 158.457 102.9237) (end 158.457 104.449644) (width 0.1) (layer "F.Cu") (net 25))
 (segment (start 152.5 97.2) (end 152.54975 97.24975) (width 0.1) (layer "F.Cu") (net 13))
 (segment (start 149.75 107.049994) (end 149.399994 107.4) (width 0.1) (layer "F.Cu") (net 13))
 (segment (start 149.75 105.25) (end 149.75 107.049994) (width 0.1) (layer "F.Cu") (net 13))
 (segment (start 152.54975 97.24975) (end 152.54975 98.4923) (width 0.1) (layer "F.Cu") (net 13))
 (via (at 149.399994 107.4) (size 0.6) (drill 0.3) (layers "F.Cu" "B.Cu") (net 13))
 (via (at 152.5 97.2) (size 0.6) (drill 0.3) (layers "F.Cu" "B.Cu") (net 13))
 (segment (start 149.399994 107.4) (end 149.399994 100.300006) (width 0.1) (layer "B.Cu") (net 13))
 (segment (start 149.399994 100.300006) (end 152.5 97.2) (width 0.1) (layer "B.Cu") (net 13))
 (segment (start 156.726944 102.045) (end 157.855 103.173056) (width 0.1) (layer "F.Cu") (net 23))
 (segment (start 159.602 106.622322) (end 159.602 109.275678) (width 0.1) (layer "F.Cu") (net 23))
 (segment (start 159.602 109.275678) (end 159.425678 109.452) (width 0.1) (layer "F.Cu") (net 23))
 (segment (start 156.702 109.452) (end 153.25 106) (width 0.1) (layer "F.Cu") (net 23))
 (segment (start 153.5 102.844) (end 154.299 102.045) (width 0.1) (layer "F.Cu") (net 23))
 (segment (start 154.299 102.045) (end 156.726944 102.045) (width 0.1) (layer "F.Cu") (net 23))
 (segment (start 148.73975 102.43975) (end 149.144 102.844) (width 0.1) (layer "F.Cu") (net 23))
 (segment (start 157.855 103.173056) (end 157.855 104.875322) (width 0.1) (layer "F.Cu") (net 23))
 (segment (start 153.25 106) (end 153.25 105.25) (width 0.1) (layer "F.Cu") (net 23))
 (segment (start 157.855 104.875322) (end 159.602 106.622322) (width 0.1) (layer "F.Cu") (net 23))
 (segment (start 149.144 102.844) (end 153.5 102.844) (width 0.1) (layer "F.Cu") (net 23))
 (segment (start 159.425678 109.452) (end 156.702 109.452) (width 0.1) (layer "F.Cu") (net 23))
 (segment (start 148.73975 99.4321) (end 148.73975 102.43975) (width 0.1) (layer "F.Cu") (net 23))
 (segment (start 155.651 104.349) (end 155.75 104.448) (width 0.1) (layer "F.Cu") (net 18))
 (segment (start 145.56475 99.4321) (end 145.56475 103.91375) (width 0.1) (layer "F.Cu") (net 18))
 (segment (start 146 104.349) (end 155.651 104.349) (width 0.1) (layer "F.Cu") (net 18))
 (segment (start 155.75 104.448) (end 155.75 105.25) (width 0.1) (layer "F.Cu") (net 18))
 (segment (start 145.56475 103.91375) (end 146 104.349) (width 0.1) (layer "F.Cu") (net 18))
 (segment (start 156.477588 102.647) (end 157.253 103.422412) (width 0.1) (layer "F.Cu") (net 21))
 (segment (start 148 103.446) (end 153.750644 103.446) (width 0.1) (layer "F.Cu") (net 21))
 (segment (start 156.751356 106.8) (end 154.998 106.8) (width 0.1) (layer "F.Cu") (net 21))
 (segment (start 154.998 106.8) (end 154.25 106.052) (width 0.1) (layer "F.Cu") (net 21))
 (segment (start 154.549644 102.647) (end 156.477588 102.647) (width 0.1) (layer "F.Cu") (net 21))
 (segment (start 147.46975 102.91575) (end 148 103.446) (width 0.1) (layer "F.Cu") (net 21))
 (segment (start 157.253 103.422412) (end 157.253 106.298356) (width 0.1) (layer "F.Cu") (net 21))
 (segment (start 154.25 106.052) (end 154.25 105.25) (width 0.1) (layer "F.Cu") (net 21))
 (segment (start 153.750644 103.446) (end 154.549644 102.647) (width 0.1) (layer "F.Cu") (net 21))
 (segment (start 147.46975 99.4321) (end 147.46975 102.91575) (width 0.1) (layer "F.Cu") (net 21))
 (segment (start 157.253 106.298356) (end 156.751356 106.8) (width 0.1) (layer "F.Cu") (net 21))
 (segment (start 139.194 109.77439) (end 139.194 106.22561) (width 0.1) (layer "F.Cu") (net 11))
 (segment (start 140.668966 97.848482) (end 143.424448 95.093) (width 0.1) (layer "F.Cu") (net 11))
 (segment (start 148.75 106.052) (end 144.146 110.656) (width 0.1) (layer "F.Cu") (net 11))
 (segment (start 148.31895 95.093) (end 151.27975 98.0538) (width 0.1) (layer "F.Cu") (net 11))
 (segment (start 140.07561 110.656) (end 139.194 109.77439) (width 0.1) (layer "F.Cu") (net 11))
 (segment (start 140.668966 104.750644) (end 140.668966 97.848482) (width 0.1) (layer "F.Cu") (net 11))
 (segment (start 151.27975 98.0538) (end 151.27975 98.4923) (width 0.1) (layer "F.Cu") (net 11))
 (segment (start 139.194 106.22561) (end 140.668966 104.750644) (width 0.1) (layer "F.Cu") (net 11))
 (segment (start 148.75 105.25) (end 148.75 106.052) (width 0.1) (layer "F.Cu") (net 11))
 (segment (start 144.146 110.656) (end 140.07561 110.656) (width 0.1) (layer "F.Cu") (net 11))
 (segment (start 143.424448 95.093) (end 148.31895 95.093) (width 0.1) (layer "F.Cu") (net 11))
 (segment (start 143.149 98.773872) (end 144.363572 97.5593) (width 0.1) (layer "F.Cu") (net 3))
 (segment (start 144.75 105.25) (end 144.75 106.052) (width 0.1) (layer "F.Cu") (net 3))
 (segment (start 144.651 106.151) (end 143.349 106.151) (width 0.1) (layer "F.Cu") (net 3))
 (segment (start 144.363572 97.5593) (end 145.70525 97.5593) (width 0.1) (layer "F.Cu") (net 3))
 (segment (start 145.70525 97.5593) (end 146.19975 98.0538) (width 0.1) (layer "F.Cu") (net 3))
 (segment (start 146.19975 98.0538) (end 146.19975 98.4923) (width 0.1) (layer "F.Cu") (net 3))
 (segment (start 143.349 106.151) (end 143.149 105.951) (width 0.1) (layer "F.Cu") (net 3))
 (segment (start 143.149 105.951) (end 143.149 98.773872) (width 0.1) (layer "F.Cu") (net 3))
 (segment (start 144.75 106.052) (end 144.651 106.151) (width 0.1) (layer "F.Cu") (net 3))
 (segment (start 148.10475 102.74975) (end 148.5 103.145) (width 0.1) (layer "F.Cu") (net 22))
 (segment (start 148.5 103.145) (end 153.625966 103.145) (width 0.1) (layer "F.Cu") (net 22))
 (segment (start 157.554 103.297734) (end 157.554 105) (width 0.1) (layer "F.Cu") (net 22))
 (segment (start 157.554 105) (end 159.301 106.747) (width 0.1) (layer "F.Cu") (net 22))
 (segment (start 153.75 105.977678) (end 153.75 105.25) (width 0.1) (layer "F.Cu") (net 22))
 (segment (start 156.923322 109.151) (end 153.75 105.977678) (width 0.1) (layer "F.Cu") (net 22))
 (segment (start 159.301 109.151) (end 156.923322 109.151) (width 0.1) (layer "F.Cu") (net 22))
 (segment (start 159.301 106.747) (end 159.301 109.151) (width 0.1) (layer "F.Cu") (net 22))
 (segment (start 154.424966 102.346) (end 156.602266 102.346) (width 0.1) (layer "F.Cu") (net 22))
 (segment (start 148.10475 99.4321) (end 148.10475 102.74975) (width 0.1) (layer "F.Cu") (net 22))
 (segment (start 156.602266 102.346) (end 157.554 103.297734) (width 0.1) (layer "F.Cu") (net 22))
 (segment (start 153.625966 103.145) (end 154.424966 102.346) (width 0.1) (layer "F.Cu") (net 22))
 (segment (start 147.35945 95.996) (end 149.37475 98.0113) (width 0.1) (layer "F.Cu") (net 8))
 (segment (start 141.644 105.454) (end 141.644 98.150482) (width 0.1) (layer "F.Cu") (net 8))
 (segment (start 141.5 105.598) (end 141.644 105.454) (width 0.1) (layer "F.Cu") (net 8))
 (segment (start 147.25 106.052) (end 143.549 109.753) (width 0.1) (layer "F.Cu") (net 8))
 (segment (start 143.549 109.753) (end 140.449644 109.753) (width 0.1) (layer "F.Cu") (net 8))
 (segment (start 149.37475 98.0113) (end 149.37475 98.4923) (width 0.1) (layer "F.Cu") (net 8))
 (segment (start 141.098644 105.598) (end 141.5 105.598) (width 0.1) (layer "F.Cu") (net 8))
 (segment (start 140.449644 109.753) (end 140.097 109.400356) (width 0.1) (layer "F.Cu") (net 8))
 (segment (start 143.798482 95.996) (end 147.35945 95.996) (width 0.1) (layer "F.Cu") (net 8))
 (segment (start 147.25 105.25) (end 147.25 106.052) (width 0.1) (layer "F.Cu") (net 8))
 (segment (start 140.097 106.599644) (end 141.098644 105.598) (width 0.1) (layer "F.Cu") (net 8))
 (segment (start 140.097 109.400356) (end 140.097 106.599644) (width 0.1) (layer "F.Cu") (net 8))
 (segment (start 141.644 98.150482) (end 143.798482 95.996) (width 0.1) (layer "F.Cu") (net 8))
 (segment (start 156.228232 103.249) (end 156.651 103.671768) (width 0.1) (layer "F.Cu") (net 19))
 (segment (start 146.19975 103.74775) (end 146.5 104.048) (width 0.1) (layer "F.Cu") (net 19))
 (segment (start 154 104.048) (end 154.799 103.249) (width 0.1) (layer "F.Cu") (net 19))
 (segment (start 156.651 106.049) (end 156.549 106.151) (width 0.1) (layer "F.Cu") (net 19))
 (segment (start 146.5 104.048) (end 154 104.048) (width 0.1) (layer "F.Cu") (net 19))
 (segment (start 154.799 103.249) (end 156.228232 103.249) (width 0.1) (layer "F.Cu") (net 19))
 (segment (start 156.651 103.671768) (end 156.651 106.049) (width 0.1) (layer "F.Cu") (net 19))
 (segment (start 156.549 106.151) (end 155.349 106.151) (width 0.1) (layer "F.Cu") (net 19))
 (segment (start 146.19975 99.4321) (end 146.19975 103.74775) (width 0.1) (layer "F.Cu") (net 19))
 (segment (start 155.349 106.151) (end 155.25 106.052) (width 0.1) (layer "F.Cu") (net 19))
 (segment (start 155.25 106.052) (end 155.25 105.25) (width 0.1) (layer "F.Cu") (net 19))
 (segment (start 153.125966 101.941) (end 153.924966 101.142) (width 0.1) (layer "F.Cu") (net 26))
 (segment (start 158.758 102.799022) (end 158.758 104.324966) (width 0.1) (layer "F.Cu") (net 26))
 (segment (start 156.105 110.355) (end 151.75 106) (width 0.1) (layer "F.Cu") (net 26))
 (segment (start 150.64475 99.4321) (end 150.64475 101.58575) (width 0.1) (layer "F.Cu") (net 26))
 (segment (start 153.924966 101.142) (end 157.100978 101.142) (width 0.1) (layer "F.Cu") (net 26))
 (segment (start 150.64475 101.58575) (end 151 101.941) (width 0.1) (layer "F.Cu") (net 26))
 (segment (start 151 101.941) (end 153.125966 101.941) (width 0.1) (layer "F.Cu") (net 26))
 (segment (start 157.100978 101.142) (end 158.758 102.799022) (width 0.1) (layer "F.Cu") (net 26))
 (segment (start 159.799712 110.355) (end 156.105 110.355) (width 0.1) (layer "F.Cu") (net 26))
 (segment (start 151.75 106) (end 151.75 105.25) (width 0.1) (layer "F.Cu") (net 26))
 (segment (start 160.505 106.071966) (end 160.505 109.649712) (width 0.1) (layer "F.Cu") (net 26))
 (segment (start 158.758 104.324966) (end 160.505 106.071966) (width 0.1) (layer "F.Cu") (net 26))
 (segment (start 160.505 109.649712) (end 159.799712 110.355) (width 0.1) (layer "F.Cu") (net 26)))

